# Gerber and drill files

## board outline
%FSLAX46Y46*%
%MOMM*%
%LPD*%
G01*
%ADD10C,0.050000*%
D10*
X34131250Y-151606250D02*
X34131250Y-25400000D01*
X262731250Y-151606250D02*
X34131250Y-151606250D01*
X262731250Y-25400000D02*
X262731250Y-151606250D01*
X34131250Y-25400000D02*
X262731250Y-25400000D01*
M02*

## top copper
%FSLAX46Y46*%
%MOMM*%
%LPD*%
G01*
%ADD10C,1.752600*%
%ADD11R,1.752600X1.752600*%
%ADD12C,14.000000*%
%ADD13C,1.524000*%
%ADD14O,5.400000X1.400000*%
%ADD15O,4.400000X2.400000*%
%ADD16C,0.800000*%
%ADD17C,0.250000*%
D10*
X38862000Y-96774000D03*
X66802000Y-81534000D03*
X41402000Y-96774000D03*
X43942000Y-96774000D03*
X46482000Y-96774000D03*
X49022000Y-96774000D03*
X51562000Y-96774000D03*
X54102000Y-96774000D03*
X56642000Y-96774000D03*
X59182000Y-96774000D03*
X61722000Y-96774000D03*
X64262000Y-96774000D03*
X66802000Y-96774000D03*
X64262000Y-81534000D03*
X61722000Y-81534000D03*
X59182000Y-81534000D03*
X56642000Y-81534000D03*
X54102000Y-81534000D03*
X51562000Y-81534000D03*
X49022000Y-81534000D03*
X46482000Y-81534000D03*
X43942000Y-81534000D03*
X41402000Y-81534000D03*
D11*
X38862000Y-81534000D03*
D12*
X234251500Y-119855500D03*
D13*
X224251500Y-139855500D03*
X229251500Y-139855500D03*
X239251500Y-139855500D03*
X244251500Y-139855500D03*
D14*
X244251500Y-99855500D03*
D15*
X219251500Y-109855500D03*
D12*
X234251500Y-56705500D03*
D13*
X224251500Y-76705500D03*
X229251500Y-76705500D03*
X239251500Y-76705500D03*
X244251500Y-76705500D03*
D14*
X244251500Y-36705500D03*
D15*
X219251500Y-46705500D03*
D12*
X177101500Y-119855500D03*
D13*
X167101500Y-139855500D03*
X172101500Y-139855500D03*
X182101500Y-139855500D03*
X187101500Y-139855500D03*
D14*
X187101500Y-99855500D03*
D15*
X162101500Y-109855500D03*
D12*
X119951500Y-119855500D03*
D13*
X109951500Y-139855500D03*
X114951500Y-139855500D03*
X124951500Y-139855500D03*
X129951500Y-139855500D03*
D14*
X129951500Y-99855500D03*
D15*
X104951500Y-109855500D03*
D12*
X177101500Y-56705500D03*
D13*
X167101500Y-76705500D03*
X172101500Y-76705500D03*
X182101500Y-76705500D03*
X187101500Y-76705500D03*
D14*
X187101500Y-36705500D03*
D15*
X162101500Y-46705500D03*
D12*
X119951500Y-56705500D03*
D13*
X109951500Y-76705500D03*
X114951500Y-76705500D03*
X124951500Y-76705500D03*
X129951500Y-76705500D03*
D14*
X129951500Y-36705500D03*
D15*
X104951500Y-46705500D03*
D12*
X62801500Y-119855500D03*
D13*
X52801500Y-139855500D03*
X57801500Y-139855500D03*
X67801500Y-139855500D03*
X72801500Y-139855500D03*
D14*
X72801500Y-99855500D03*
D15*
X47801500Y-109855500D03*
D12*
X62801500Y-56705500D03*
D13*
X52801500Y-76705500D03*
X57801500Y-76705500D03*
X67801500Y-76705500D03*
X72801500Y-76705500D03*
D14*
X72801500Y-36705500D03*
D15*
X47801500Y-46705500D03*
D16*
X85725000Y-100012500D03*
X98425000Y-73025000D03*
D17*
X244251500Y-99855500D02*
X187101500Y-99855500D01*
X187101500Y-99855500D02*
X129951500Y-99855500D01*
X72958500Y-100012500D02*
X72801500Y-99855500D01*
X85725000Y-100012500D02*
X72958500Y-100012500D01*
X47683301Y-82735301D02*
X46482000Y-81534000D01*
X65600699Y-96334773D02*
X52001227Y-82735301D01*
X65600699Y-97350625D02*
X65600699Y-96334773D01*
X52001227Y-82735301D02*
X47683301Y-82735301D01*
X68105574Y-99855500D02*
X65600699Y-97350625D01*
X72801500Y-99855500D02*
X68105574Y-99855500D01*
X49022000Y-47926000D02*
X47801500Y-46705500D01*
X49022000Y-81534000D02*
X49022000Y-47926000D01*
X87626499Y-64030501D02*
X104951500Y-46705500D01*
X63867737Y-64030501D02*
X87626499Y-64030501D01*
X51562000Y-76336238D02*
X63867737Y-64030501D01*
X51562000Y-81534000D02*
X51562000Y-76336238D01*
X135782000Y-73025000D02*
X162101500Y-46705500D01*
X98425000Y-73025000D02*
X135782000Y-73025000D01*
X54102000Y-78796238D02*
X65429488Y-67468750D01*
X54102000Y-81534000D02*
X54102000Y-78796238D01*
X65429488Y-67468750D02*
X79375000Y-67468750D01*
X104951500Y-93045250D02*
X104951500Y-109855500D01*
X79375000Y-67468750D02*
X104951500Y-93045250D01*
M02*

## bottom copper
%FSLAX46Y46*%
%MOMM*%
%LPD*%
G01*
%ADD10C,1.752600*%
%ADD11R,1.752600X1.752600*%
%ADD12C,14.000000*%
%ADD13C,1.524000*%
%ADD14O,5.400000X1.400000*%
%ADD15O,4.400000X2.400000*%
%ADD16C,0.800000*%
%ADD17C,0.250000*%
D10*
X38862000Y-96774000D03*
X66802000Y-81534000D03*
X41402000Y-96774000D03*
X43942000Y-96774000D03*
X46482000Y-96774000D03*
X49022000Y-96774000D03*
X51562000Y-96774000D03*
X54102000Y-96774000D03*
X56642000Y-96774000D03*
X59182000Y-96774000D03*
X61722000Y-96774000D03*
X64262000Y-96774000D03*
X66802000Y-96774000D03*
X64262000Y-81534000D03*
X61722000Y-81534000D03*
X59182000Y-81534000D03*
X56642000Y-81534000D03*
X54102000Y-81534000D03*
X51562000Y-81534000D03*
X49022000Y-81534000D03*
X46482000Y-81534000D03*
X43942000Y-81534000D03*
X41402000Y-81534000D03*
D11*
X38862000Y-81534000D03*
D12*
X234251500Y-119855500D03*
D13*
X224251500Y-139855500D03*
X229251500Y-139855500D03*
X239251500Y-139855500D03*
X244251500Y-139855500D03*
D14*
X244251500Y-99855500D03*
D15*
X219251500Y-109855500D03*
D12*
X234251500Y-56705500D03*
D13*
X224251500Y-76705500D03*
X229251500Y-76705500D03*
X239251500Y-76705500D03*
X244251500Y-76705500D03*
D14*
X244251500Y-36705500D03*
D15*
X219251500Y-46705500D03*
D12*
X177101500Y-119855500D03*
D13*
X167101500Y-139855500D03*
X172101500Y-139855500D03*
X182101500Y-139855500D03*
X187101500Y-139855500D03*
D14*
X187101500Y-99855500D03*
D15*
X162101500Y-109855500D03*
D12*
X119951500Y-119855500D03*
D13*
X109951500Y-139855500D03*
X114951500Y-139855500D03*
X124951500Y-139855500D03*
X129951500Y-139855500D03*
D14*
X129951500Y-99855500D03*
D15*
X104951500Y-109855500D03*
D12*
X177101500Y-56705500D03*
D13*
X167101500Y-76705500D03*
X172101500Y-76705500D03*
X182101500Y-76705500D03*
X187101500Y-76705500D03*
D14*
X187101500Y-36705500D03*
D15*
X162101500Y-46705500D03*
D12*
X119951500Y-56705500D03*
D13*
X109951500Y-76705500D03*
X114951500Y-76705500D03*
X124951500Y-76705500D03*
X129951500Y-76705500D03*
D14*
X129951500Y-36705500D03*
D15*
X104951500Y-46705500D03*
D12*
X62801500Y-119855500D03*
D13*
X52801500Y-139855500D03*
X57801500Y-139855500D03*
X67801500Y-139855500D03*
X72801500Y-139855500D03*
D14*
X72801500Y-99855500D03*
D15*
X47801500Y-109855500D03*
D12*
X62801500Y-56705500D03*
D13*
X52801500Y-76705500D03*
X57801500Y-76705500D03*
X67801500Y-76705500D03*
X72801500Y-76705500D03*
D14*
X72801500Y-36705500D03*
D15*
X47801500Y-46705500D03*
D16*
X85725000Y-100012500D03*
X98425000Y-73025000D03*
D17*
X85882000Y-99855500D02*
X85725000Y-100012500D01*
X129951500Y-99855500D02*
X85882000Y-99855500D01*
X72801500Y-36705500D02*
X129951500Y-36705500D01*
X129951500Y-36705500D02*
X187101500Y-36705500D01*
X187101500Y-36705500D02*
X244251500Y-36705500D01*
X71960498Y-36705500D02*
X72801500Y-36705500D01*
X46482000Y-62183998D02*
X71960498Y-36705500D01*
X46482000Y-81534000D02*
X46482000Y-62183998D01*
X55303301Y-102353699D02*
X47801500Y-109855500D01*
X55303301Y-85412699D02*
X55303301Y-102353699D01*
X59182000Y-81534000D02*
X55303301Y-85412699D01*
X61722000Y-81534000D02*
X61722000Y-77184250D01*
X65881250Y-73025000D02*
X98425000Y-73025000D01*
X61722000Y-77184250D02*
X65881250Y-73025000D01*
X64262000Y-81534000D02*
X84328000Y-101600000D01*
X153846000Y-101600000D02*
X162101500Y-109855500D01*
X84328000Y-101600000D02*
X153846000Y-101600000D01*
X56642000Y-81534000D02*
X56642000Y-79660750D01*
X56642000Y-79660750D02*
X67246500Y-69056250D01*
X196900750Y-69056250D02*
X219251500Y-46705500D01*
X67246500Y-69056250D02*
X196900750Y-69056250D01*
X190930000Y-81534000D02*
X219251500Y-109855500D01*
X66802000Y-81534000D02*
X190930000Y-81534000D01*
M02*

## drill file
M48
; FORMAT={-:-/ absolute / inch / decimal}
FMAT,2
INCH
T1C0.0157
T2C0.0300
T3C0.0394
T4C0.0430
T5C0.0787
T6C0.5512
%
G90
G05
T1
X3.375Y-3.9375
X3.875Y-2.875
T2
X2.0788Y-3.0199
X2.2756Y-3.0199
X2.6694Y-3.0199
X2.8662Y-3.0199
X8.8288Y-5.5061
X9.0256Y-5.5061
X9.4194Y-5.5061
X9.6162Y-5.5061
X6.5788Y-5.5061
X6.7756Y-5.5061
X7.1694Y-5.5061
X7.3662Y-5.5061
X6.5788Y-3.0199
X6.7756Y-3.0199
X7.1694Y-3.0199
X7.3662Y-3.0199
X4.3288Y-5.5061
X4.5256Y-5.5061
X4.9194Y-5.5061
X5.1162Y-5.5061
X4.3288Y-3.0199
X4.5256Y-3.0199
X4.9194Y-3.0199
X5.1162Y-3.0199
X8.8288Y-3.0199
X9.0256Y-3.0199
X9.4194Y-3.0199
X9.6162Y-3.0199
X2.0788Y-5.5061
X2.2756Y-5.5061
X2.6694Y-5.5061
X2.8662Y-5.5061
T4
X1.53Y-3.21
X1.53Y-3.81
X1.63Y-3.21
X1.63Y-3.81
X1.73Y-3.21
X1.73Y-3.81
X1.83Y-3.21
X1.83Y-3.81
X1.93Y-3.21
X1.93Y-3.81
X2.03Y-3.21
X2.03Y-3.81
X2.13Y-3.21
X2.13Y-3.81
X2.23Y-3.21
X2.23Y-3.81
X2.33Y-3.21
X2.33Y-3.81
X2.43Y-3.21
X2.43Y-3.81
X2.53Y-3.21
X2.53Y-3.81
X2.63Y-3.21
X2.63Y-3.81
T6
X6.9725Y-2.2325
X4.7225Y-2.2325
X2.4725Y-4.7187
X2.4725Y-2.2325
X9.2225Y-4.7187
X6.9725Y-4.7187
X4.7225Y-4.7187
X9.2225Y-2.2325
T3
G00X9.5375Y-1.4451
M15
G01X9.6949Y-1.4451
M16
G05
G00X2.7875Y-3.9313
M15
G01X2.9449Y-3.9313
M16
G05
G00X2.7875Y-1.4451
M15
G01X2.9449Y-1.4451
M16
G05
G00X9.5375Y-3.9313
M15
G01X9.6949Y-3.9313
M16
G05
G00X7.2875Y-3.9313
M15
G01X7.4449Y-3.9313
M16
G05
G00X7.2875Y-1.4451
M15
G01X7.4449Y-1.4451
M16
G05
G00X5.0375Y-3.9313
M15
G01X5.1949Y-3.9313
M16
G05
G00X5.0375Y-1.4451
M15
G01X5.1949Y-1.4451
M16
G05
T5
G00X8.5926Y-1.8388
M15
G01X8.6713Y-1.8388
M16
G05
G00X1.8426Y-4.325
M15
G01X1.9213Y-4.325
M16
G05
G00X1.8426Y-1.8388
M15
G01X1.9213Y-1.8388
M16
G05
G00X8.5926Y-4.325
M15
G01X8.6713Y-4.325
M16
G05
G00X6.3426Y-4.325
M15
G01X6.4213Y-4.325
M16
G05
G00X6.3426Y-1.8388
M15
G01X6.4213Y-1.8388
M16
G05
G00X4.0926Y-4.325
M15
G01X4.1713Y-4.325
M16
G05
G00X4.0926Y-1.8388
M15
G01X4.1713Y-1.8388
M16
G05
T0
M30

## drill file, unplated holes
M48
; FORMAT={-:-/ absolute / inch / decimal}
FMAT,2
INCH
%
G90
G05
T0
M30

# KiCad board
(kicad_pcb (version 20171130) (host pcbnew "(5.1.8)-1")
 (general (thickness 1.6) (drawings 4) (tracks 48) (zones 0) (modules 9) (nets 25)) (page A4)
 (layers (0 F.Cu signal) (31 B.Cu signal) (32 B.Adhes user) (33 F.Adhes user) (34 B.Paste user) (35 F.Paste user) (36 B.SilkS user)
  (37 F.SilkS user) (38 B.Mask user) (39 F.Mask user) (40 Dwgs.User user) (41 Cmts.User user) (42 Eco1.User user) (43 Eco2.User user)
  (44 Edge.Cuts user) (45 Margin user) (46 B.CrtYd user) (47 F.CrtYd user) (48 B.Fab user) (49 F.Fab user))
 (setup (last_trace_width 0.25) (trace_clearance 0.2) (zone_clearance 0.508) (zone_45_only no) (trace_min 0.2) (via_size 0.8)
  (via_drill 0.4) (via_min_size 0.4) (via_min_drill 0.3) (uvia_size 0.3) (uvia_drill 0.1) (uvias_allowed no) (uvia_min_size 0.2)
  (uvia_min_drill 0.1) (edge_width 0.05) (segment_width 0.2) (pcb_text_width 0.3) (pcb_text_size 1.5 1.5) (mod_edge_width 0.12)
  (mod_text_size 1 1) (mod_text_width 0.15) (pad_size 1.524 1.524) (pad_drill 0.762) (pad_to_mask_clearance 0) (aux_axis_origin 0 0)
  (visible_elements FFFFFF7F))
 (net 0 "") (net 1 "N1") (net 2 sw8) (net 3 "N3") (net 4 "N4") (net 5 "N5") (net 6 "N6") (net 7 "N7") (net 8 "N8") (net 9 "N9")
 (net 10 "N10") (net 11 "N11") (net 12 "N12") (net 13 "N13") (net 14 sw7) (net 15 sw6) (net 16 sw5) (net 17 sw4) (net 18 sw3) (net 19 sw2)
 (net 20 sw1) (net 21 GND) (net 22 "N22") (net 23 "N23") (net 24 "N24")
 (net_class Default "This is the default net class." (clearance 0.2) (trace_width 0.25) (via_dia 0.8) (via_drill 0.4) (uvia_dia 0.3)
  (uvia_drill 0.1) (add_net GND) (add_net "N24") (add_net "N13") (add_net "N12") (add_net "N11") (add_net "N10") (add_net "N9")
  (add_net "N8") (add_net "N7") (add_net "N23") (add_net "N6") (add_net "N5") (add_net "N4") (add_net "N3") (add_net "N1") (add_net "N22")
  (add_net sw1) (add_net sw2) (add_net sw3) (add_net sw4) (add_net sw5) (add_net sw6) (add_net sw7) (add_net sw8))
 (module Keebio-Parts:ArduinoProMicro (layer B.Cu) (at 52.832 89.154)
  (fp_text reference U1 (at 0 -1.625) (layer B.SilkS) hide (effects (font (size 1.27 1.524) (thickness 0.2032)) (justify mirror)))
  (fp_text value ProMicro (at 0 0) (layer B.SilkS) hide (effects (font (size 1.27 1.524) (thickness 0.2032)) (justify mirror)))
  (pad 24 thru_hole circle (at -13.97 7.62) (size 1.7526 1.7526) (drill 1.0922) (layers *.Cu *.SilkS *.Mask) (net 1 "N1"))
  (pad 12 thru_hole circle (at 13.97 -7.62) (size 1.7526 1.7526) (drill 1.0922) (layers *.Cu *.SilkS *.Mask) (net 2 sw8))
  (pad 23 thru_hole circle (at -11.43 7.62) (size 1.7526 1.7526) (drill 1.0922) (layers *.Cu *.SilkS *.Mask) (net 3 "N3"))
  (pad 22 thru_hole circle (at -8.89 7.62) (size 1.7526 1.7526) (drill 1.0922) (layers *.Cu *.SilkS *.Mask) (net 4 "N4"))
  (pad 21 thru_hole circle (at -6.35 7.62) (size 1.7526 1.7526) (drill 1.0922) (layers *.Cu *.SilkS *.Mask) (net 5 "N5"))
  (pad 20 thru_hole circle (at -3.81 7.62) (size 1.7526 1.7526) (drill 1.0922) (layers *.Cu *.SilkS *.Mask) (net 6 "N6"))
  (pad 19 thru_hole circle (at -1.27 7.62) (size 1.7526 1.7526) (drill 1.0922) (layers *.Cu *.SilkS *.Mask) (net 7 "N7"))
  (pad 18 thru_hole circle (at 1.27 7.62) (size 1.7526 1.7526) (drill 1.0922) (layers *.Cu *.SilkS *.Mask) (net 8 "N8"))
  (pad 17 thru_hole circle (at 3.81 7.62) (size 1.7526 1.7526) (drill 1.0922) (layers *.Cu *.SilkS *.Mask) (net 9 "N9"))
  (pad 16 thru_hole circle (at 6.35 7.62) (size 1.7526 1.7526) (drill 1.0922) (layers *.Cu *.SilkS *.Mask) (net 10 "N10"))
  (pad 15 thru_hole circle (at 8.89 7.62) (size 1.7526 1.7526) (drill 1.0922) (layers *.Cu *.SilkS *.Mask) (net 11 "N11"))
  (pad 14 thru_hole circle (at 11.43 7.62) (size 1.7526 1.7526) (drill 1.0922) (layers *.Cu *.SilkS *.Mask) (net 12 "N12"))
  (pad 13 thru_hole circle (at 13.97 7.62) (size 1.7526 1.7526) (drill 1.0922) (layers *.Cu *.SilkS *.Mask) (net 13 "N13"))
  (pad 11 thru_hole circle (at 11.43 -7.62) (size 1.7526 1.7526) (drill 1.0922) (layers *.Cu *.SilkS *.Mask) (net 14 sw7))
  (pad 10 thru_hole circle (at 8.89 -7.62) (size 1.7526 1.7526) (drill 1.0922) (layers *.Cu *.SilkS *.Mask) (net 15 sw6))
  (pad 9 thru_hole circle (at 6.35 -7.62) (size 1.7526 1.7526) (drill 1.0922) (layers *.Cu *.SilkS *.Mask) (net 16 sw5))
  (pad 8 thru_hole circle (at 3.81 -7.62) (size 1.7526 1.7526) (drill 1.0922) (layers *.Cu *.SilkS *.Mask) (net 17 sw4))
  (pad 7 thru_hole circle (at 1.27 -7.62) (size 1.7526 1.7526) (drill 1.0922) (layers *.Cu *.SilkS *.Mask) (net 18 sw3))
  (pad 6 thru_hole circle (at -1.27 -7.62) (size 1.7526 1.7526) (drill 1.0922) (layers *.Cu *.SilkS *.Mask) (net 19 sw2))
  (pad 5 thru_hole circle (at -3.81 -7.62) (size 1.7526 1.7526) (drill 1.0922) (layers *.Cu *.SilkS *.Mask) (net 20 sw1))
  (pad 4 thru_hole circle (at -6.35 -7.62) (size 1.7526 1.7526) (drill 1.0922) (layers *.Cu *.SilkS *.Mask) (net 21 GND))
  (pad 3 thru_hole circle (at -8.89 -7.62) (size 1.7526 1.7526) (drill 1.0922) (layers *.Cu *.SilkS *.Mask) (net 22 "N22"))
  (pad 2 thru_hole circle (at -11.43 -7.62) (size 1.7526 1.7526) (drill 1.0922) (layers *.Cu *.SilkS *.Mask) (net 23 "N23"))
  (pad 1 thru_hole rect (at -13.97 -7.62) (size 1.7526 1.7526) (drill 1.0922) (layers *.Cu *.SilkS *.Mask) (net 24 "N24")))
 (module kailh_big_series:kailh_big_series (layer F.Cu) (at 234.2515 119.8555)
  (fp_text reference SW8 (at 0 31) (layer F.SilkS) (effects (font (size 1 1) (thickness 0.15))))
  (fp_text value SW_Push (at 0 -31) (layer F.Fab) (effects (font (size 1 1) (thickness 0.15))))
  (pad "" thru_hole circle (at 0 0) (size 14 14) (drill 14) (layers *.Cu *.Mask))
  (pad 7 thru_hole circle (at -10 20) (size 1.524 1.524) (drill 0.762) (layers *.Cu *.Mask))
  (pad 6 thru_hole circle (at -5 20) (size 1.524 1.524) (drill 0.762) (layers *.Cu *.Mask))
  (pad 5 thru_hole circle (at 5 20) (size 1.524 1.524) (drill 0.762) (layers *.Cu *.Mask))
  (pad 4 thru_hole circle (at 10 20) (size 1.524 1.524) (drill 0.762) (layers *.Cu *.Mask))
  (pad 2 thru_hole oval (at 10 -20) (size 5.4 1.4) (drill oval 5 1) (layers *.Cu *.Mask) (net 21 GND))
  (pad 1 thru_hole oval (at -15 -10) (size 4.4 2.4) (drill oval 4 2) (layers *.Cu *.Mask) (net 2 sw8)))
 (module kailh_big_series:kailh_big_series (layer F.Cu) (at 234.2515 56.7055)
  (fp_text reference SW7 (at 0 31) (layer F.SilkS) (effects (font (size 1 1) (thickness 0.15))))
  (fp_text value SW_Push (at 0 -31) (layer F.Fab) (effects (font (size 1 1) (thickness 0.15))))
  (pad "" thru_hole circle (at 0 0) (size 14 14) (drill 14) (layers *.Cu *.Mask))
  (pad 7 thru_hole circle (at -10 20) (size 1.524 1.524) (drill 0.762) (layers *.Cu *.Mask))
  (pad 6 thru_hole circle (at -5 20) (size 1.524 1.524) (drill 0.762) (layers *.Cu *.Mask))
  (pad 5 thru_hole circle (at 5 20) (size 1.524 1.524) (drill 0.762) (layers *.Cu *.Mask))
  (pad 4 thru_hole circle (at 10 20) (size 1.524 1.524) (drill 0.762) (layers *.Cu *.Mask))
  (pad 2 thru_hole oval (at 10 -20) (size 5.4 1.4) (drill oval 5 1) (layers *.Cu *.Mask) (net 21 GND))
  (pad 1 thru_hole oval (at -15 -10) (size 4.4 2.4) (drill oval 4 2) (layers *.Cu *.Mask) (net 17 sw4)))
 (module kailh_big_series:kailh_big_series (layer F.Cu) (at 177.1015 119.8555)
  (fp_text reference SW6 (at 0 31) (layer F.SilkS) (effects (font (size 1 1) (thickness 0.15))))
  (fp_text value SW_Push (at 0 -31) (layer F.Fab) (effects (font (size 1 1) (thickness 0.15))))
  (pad "" thru_hole circle (at 0 0) (size 14 14) (drill 14) (layers *.Cu *.Mask))
  (pad 7 thru_hole circle (at -10 20) (size 1.524 1.524) (drill 0.762) (layers *.Cu *.Mask))
  (pad 6 thru_hole circle (at -5 20) (size 1.524 1.524) (drill 0.762) (layers *.Cu *.Mask))
  (pad 5 thru_hole circle (at 5 20) (size 1.524 1.524) (drill 0.762) (layers *.Cu *.Mask))
  (pad 4 thru_hole circle (at 10 20) (size 1.524 1.524) (drill 0.762) (layers *.Cu *.Mask))
  (pad 2 thru_hole oval (at 10 -20) (size 5.4 1.4) (drill oval 5 1) (layers *.Cu *.Mask) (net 21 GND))
  (pad 1 thru_hole oval (at -15 -10) (size 4.4 2.4) (drill oval 4 2) (layers *.Cu *.Mask) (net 14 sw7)))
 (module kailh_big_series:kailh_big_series (layer F.Cu) (at 119.9515 119.8555)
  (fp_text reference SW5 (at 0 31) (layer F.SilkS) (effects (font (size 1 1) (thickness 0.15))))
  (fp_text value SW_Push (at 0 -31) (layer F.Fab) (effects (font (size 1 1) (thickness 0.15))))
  (pad "" thru_hole circle (at 0 0) (size 14 14) (drill 14) (layers *.Cu *.Mask))
  (pad 7 thru_hole circle (at -10 20) (size 1.524 1.524) (drill 0.762) (layers *.Cu *.Mask))
  (pad 6 thru_hole circle (at -5 20) (size 1.524 1.524) (drill 0.762) (layers *.Cu *.Mask))
  (pad 5 thru_hole circle (at 5 20) (size 1.524 1.524) (drill 0.762) (layers *.Cu *.Mask))
  (pad 4 thru_hole circle (at 10 20) (size 1.524 1.524) (drill 0.762) (layers *.Cu *.Mask))
  (pad 2 thru_hole oval (at 10 -20) (size 5.4 1.4) (drill oval 5 1) (layers *.Cu *.Mask) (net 21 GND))
  (pad 1 thru_hole oval (at -15 -10) (size 4.4 2.4) (drill oval 4 2) (layers *.Cu *.Mask) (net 18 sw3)))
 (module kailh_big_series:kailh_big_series (layer F.Cu) (at 177.1015 56.7055)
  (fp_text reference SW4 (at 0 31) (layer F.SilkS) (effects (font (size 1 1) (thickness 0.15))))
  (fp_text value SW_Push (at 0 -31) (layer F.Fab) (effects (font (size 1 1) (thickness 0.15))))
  (pad "" thru_hole circle (at 0 0) (size 14 14) (drill 14) (layers *.Cu *.Mask))
  (pad 7 thru_hole circle (at -10 20) (size 1.524 1.524) (drill 0.762) (layers *.Cu *.Mask))
  (pad 6 thru_hole circle (at -5 20) (size 1.524 1.524) (drill 0.762) (layers *.Cu *.Mask))
  (pad 5 thru_hole circle (at 5 20) (size 1.524 1.524) (drill 0.762) (layers *.Cu *.Mask))
  (pad 4 thru_hole circle (at 10 20) (size 1.524 1.524) (drill 0.762) (layers *.Cu *.Mask))
  (pad 2 thru_hole oval (at 10 -20) (size 5.4 1.4) (drill oval 5 1) (layers *.Cu *.Mask) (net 21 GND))
  (pad 1 thru_hole oval (at -15 -10) (size 4.4 2.4) (drill oval 4 2) (layers *.Cu *.Mask) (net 15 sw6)))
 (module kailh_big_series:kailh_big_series (layer F.Cu) (at 119.9515 56.7055)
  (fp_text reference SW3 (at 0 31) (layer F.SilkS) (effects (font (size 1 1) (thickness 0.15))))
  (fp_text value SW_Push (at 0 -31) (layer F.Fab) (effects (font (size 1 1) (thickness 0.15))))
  (pad "" thru_hole circle (at 0 0) (size 14 14) (drill 14) (layers *.Cu *.Mask))
  (pad 7 thru_hole circle (at -10 20) (size 1.524 1.524) (drill 0.762) (layers *.Cu *.Mask))
  (pad 6 thru_hole circle (at -5 20) (size 1.524 1.524) (drill 0.762) (layers *.Cu *.Mask))
  (pad 5 thru_hole circle (at 5 20) (size 1.524 1.524) (drill 0.762) (layers *.Cu *.Mask))
  (pad 4 thru_hole circle (at 10 20) (size 1.524 1.524) (drill 0.762) (layers *.Cu *.Mask))
  (pad 2 thru_hole oval (at 10 -20) (size 5.4 1.4) (drill oval 5 1) (layers *.Cu *.Mask) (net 21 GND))
  (pad 1 thru_hole oval (at -15 -10) (size 4.4 2.4) (drill oval 4 2) (layers *.Cu *.Mask) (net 19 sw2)))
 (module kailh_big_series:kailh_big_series (layer F.Cu) (at 62.8015 119.8555)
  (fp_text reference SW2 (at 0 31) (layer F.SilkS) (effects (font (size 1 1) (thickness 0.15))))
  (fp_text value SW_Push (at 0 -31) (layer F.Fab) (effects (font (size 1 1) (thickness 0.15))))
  (pad "" thru_hole circle (at 0 0) (size 14 14) (drill 14) (layers *.Cu *.Mask))
  (pad 7 thru_hole circle (at -10 20) (size 1.524 1.524) (drill 0.762) (layers *.Cu *.Mask))
  (pad 6 thru_hole circle (at -5 20) (size 1.524 1.524) (drill 0.762) (layers *.Cu *.Mask))
  (pad 5 thru_hole circle (at 5 20) (size 1.524 1.524) (drill 0.762) (layers *.Cu *.Mask))
  (pad 4 thru_hole circle (at 10 20) (size 1.524 1.524) (drill 0.762) (layers *.Cu *.Mask))
  (pad 2 thru_hole oval (at 10 -20) (size 5.4 1.4) (drill oval 5 1) (layers *.Cu *.Mask) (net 21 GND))
  (pad 1 thru_hole oval (at -15 -10) (size 4.4 2.4) (drill oval 4 2) (layers *.Cu *.Mask) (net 16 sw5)))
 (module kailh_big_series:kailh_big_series (layer F.Cu) (at 62.8015 56.7055)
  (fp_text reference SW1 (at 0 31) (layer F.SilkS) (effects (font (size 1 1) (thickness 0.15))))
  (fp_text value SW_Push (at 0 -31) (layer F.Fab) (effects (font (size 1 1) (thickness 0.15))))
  (pad "" thru_hole circle (at 0 0) (size 14 14) (drill 14) (layers *.Cu *.Mask))
  (pad 7 thru_hole circle (at -10 20) (size 1.524 1.524) (drill 0.762) (layers *.Cu *.Mask))
  (pad 6 thru_hole circle (at -5 20) (size 1.524 1.524) (drill 0.762) (layers *.Cu *.Mask))
  (pad 5 thru_hole circle (at 5 20) (size 1.524 1.524) (drill 0.762) (layers *.Cu *.Mask))
  (pad 4 thru_hole circle (at 10 20) (size 1.524 1.524) (drill 0.762) (layers *.Cu *.Mask))
  (pad 2 thru_hole oval (at 10 -20) (size 5.4 1.4) (drill oval 5 1) (layers *.Cu *.Mask) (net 21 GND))
  (pad 1 thru_hole oval (at -15 -10) (size 4.4 2.4) (drill oval 4 2) (layers *.Cu *.Mask) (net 20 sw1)))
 (gr_line (start 34.13125 151.60625) (end 34.13125 25.4) (layer Edge.Cuts) (width 0.05))
 (gr_line (start 262.73125 151.60625) (end 34.13125 151.60625) (layer Edge.Cuts) (width 0.05))
 (gr_line (start 262.73125 25.4) (end 262.73125 151.60625) (layer Edge.Cuts) (width 0.05))
 (gr_line (start 34.13125 25.4) (end 262.73125 25.4) (layer Edge.Cuts) (width 0.05))
 (segment (start 244.2515 99.8555) (end 187.1015 99.8555) (width 0.25) (layer F.Cu) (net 21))
 (segment (start 187.1015 99.8555) (end 129.9515 99.8555) (width 0.25) (layer F.Cu) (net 21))
 (via (at 85.725 100.0125) (size 0.8) (drill 0.4) (layers F.Cu B.Cu) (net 21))
 (segment (start 85.882 99.8555) (end 85.725 100.0125) (width 0.25) (layer B.Cu) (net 21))
 (segment (start 129.9515 99.8555) (end 85.882 99.8555) (width 0.25) (layer B.Cu) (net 21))
 (segment (start 72.9585 100.0125) (end 72.8015 99.8555) (width 0.25) (layer F.Cu) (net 21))
 (segment (start 85.725 100.0125) (end 72.9585 100.0125) (width 0.25) (layer F.Cu) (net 21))
 (segment (start 72.8015 36.7055) (end 129.9515 36.7055) (width 0.25) (layer B.Cu) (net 21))
 (segment (start 129.9515 36.7055) (end 187.1015 36.7055) (width 0.25) (layer B.Cu) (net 21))
 (segment (start 187.1015 36.7055) (end 244.2515 36.7055) (width 0.25) (layer B.Cu) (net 21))
 (segment (start 71.960498 36.7055) (end 72.8015 36.7055) (width 0.25) (layer B.Cu) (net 21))
 (segment (start 46.482 62.183998) (end 71.960498 36.7055) (width 0.25) (layer B.Cu) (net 21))
 (segment (start 46.482 81.534) (end 46.482 62.183998) (width 0.25) (layer B.Cu) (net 21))
 (segment (start 47.683301 82.735301) (end 46.482 81.534) (width 0.25) (layer F.Cu) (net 21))
 (segment (start 65.600699 96.334773) (end 52.001227 82.735301) (width 0.25) (layer F.Cu) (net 21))
 (segment (start 65.600699 97.350625) (end 65.600699 96.334773) (width 0.25) (layer F.Cu) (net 21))
 (segment (start 52.001227 82.735301) (end 47.683301 82.735301) (width 0.25) (layer F.Cu) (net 21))
 (segment (start 68.105574 99.8555) (end 65.600699 97.350625) (width 0.25) (layer F.Cu) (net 21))
 (segment (start 72.8015 99.8555) (end 68.105574 99.8555) (width 0.25) (layer F.Cu) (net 21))
 (segment (start 49.022 47.926) (end 47.8015 46.7055) (width 0.25) (layer F.Cu) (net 20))
 (segment (start 49.022 81.534) (end 49.022 47.926) (width 0.25) (layer F.Cu) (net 20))
 (segment (start 55.303301 102.353699) (end 47.8015 109.8555) (width 0.25) (layer B.Cu) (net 16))
 (segment (start 55.303301 85.412699) (end 55.303301 102.353699) (width 0.25) (layer B.Cu) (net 16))
 (segment (start 59.182 81.534) (end 55.303301 85.412699) (width 0.25) (layer B.Cu) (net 16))
 (segment (start 87.626499 64.030501) (end 104.9515 46.7055) (width 0.25) (layer F.Cu) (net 19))
 (segment (start 63.867737 64.030501) (end 87.626499 64.030501) (width 0.25) (layer F.Cu) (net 19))
 (segment (start 51.562 76.336238) (end 63.867737 64.030501) (width 0.25) (layer F.Cu) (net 19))
 (segment (start 51.562 81.534) (end 51.562 76.336238) (width 0.25) (layer F.Cu) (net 19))
 (segment (start 61.722 81.534) (end 61.722 77.18425) (width 0.25) (layer B.Cu) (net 15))
 (via (at 98.425 73.025) (size 0.8) (drill 0.4) (layers F.Cu B.Cu) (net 15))
 (segment (start 65.88125 73.025) (end 98.425 73.025) (width 0.25) (layer B.Cu) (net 15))
 (segment (start 61.722 77.18425) (end 65.88125 73.025) (width 0.25) (layer B.Cu) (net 15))
 (segment (start 135.782 73.025) (end 162.1015 46.7055) (width 0.25) (layer F.Cu) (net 15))
 (segment (start 98.425 73.025) (end 135.782 73.025) (width 0.25) (layer F.Cu) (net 15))
 (segment (start 54.102 78.796238) (end 65.429488 67.46875) (width 0.25) (layer F.Cu) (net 18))
 (segment (start 54.102 81.534) (end 54.102 78.796238) (width 0.25) (layer F.Cu) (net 18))
 (segment (start 65.429488 67.46875) (end 79.375 67.46875) (width 0.25) (layer F.Cu) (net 18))
 (segment (start 104.9515 93.04525) (end 104.9515 109.8555) (width 0.25) (layer F.Cu) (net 18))
 (segment (start 79.375 67.46875) (end 104.9515 93.04525) (width 0.25) (layer F.Cu) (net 18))
 (segment (start 64.262 81.534) (end 84.328 101.6) (width 0.25) (layer B.Cu) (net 14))
 (segment (start 153.846 101.6) (end 162.1015 109.8555) (width 0.25) (layer B.Cu) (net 14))
 (segment (start 84.328 101.6) (end 153.846 101.6) (width 0.25) (layer B.Cu) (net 14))
 (segment (start 56.642 81.534) (end 56.642 79.66075) (width 0.25) (layer B.Cu) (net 17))
 (segment (start 56.642 79.66075) (end 67.2465 69.05625) (width 0.25) (layer B.Cu) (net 17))
 (segment (start 196.90075 69.05625) (end 219.2515 46.7055) (width 0.25) (layer B.Cu) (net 17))
 (segment (start 67.2465 69.05625) (end 196.90075 69.05625) (width 0.25) (layer B.Cu) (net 17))
 (segment (start 190.93 81.534) (end 219.2515 109.8555) (width 0.25) (layer B.Cu) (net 2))
 (segment (start 66.802 81.534) (end 190.93 81.534) (width 0.25) (layer B.Cu) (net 2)))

